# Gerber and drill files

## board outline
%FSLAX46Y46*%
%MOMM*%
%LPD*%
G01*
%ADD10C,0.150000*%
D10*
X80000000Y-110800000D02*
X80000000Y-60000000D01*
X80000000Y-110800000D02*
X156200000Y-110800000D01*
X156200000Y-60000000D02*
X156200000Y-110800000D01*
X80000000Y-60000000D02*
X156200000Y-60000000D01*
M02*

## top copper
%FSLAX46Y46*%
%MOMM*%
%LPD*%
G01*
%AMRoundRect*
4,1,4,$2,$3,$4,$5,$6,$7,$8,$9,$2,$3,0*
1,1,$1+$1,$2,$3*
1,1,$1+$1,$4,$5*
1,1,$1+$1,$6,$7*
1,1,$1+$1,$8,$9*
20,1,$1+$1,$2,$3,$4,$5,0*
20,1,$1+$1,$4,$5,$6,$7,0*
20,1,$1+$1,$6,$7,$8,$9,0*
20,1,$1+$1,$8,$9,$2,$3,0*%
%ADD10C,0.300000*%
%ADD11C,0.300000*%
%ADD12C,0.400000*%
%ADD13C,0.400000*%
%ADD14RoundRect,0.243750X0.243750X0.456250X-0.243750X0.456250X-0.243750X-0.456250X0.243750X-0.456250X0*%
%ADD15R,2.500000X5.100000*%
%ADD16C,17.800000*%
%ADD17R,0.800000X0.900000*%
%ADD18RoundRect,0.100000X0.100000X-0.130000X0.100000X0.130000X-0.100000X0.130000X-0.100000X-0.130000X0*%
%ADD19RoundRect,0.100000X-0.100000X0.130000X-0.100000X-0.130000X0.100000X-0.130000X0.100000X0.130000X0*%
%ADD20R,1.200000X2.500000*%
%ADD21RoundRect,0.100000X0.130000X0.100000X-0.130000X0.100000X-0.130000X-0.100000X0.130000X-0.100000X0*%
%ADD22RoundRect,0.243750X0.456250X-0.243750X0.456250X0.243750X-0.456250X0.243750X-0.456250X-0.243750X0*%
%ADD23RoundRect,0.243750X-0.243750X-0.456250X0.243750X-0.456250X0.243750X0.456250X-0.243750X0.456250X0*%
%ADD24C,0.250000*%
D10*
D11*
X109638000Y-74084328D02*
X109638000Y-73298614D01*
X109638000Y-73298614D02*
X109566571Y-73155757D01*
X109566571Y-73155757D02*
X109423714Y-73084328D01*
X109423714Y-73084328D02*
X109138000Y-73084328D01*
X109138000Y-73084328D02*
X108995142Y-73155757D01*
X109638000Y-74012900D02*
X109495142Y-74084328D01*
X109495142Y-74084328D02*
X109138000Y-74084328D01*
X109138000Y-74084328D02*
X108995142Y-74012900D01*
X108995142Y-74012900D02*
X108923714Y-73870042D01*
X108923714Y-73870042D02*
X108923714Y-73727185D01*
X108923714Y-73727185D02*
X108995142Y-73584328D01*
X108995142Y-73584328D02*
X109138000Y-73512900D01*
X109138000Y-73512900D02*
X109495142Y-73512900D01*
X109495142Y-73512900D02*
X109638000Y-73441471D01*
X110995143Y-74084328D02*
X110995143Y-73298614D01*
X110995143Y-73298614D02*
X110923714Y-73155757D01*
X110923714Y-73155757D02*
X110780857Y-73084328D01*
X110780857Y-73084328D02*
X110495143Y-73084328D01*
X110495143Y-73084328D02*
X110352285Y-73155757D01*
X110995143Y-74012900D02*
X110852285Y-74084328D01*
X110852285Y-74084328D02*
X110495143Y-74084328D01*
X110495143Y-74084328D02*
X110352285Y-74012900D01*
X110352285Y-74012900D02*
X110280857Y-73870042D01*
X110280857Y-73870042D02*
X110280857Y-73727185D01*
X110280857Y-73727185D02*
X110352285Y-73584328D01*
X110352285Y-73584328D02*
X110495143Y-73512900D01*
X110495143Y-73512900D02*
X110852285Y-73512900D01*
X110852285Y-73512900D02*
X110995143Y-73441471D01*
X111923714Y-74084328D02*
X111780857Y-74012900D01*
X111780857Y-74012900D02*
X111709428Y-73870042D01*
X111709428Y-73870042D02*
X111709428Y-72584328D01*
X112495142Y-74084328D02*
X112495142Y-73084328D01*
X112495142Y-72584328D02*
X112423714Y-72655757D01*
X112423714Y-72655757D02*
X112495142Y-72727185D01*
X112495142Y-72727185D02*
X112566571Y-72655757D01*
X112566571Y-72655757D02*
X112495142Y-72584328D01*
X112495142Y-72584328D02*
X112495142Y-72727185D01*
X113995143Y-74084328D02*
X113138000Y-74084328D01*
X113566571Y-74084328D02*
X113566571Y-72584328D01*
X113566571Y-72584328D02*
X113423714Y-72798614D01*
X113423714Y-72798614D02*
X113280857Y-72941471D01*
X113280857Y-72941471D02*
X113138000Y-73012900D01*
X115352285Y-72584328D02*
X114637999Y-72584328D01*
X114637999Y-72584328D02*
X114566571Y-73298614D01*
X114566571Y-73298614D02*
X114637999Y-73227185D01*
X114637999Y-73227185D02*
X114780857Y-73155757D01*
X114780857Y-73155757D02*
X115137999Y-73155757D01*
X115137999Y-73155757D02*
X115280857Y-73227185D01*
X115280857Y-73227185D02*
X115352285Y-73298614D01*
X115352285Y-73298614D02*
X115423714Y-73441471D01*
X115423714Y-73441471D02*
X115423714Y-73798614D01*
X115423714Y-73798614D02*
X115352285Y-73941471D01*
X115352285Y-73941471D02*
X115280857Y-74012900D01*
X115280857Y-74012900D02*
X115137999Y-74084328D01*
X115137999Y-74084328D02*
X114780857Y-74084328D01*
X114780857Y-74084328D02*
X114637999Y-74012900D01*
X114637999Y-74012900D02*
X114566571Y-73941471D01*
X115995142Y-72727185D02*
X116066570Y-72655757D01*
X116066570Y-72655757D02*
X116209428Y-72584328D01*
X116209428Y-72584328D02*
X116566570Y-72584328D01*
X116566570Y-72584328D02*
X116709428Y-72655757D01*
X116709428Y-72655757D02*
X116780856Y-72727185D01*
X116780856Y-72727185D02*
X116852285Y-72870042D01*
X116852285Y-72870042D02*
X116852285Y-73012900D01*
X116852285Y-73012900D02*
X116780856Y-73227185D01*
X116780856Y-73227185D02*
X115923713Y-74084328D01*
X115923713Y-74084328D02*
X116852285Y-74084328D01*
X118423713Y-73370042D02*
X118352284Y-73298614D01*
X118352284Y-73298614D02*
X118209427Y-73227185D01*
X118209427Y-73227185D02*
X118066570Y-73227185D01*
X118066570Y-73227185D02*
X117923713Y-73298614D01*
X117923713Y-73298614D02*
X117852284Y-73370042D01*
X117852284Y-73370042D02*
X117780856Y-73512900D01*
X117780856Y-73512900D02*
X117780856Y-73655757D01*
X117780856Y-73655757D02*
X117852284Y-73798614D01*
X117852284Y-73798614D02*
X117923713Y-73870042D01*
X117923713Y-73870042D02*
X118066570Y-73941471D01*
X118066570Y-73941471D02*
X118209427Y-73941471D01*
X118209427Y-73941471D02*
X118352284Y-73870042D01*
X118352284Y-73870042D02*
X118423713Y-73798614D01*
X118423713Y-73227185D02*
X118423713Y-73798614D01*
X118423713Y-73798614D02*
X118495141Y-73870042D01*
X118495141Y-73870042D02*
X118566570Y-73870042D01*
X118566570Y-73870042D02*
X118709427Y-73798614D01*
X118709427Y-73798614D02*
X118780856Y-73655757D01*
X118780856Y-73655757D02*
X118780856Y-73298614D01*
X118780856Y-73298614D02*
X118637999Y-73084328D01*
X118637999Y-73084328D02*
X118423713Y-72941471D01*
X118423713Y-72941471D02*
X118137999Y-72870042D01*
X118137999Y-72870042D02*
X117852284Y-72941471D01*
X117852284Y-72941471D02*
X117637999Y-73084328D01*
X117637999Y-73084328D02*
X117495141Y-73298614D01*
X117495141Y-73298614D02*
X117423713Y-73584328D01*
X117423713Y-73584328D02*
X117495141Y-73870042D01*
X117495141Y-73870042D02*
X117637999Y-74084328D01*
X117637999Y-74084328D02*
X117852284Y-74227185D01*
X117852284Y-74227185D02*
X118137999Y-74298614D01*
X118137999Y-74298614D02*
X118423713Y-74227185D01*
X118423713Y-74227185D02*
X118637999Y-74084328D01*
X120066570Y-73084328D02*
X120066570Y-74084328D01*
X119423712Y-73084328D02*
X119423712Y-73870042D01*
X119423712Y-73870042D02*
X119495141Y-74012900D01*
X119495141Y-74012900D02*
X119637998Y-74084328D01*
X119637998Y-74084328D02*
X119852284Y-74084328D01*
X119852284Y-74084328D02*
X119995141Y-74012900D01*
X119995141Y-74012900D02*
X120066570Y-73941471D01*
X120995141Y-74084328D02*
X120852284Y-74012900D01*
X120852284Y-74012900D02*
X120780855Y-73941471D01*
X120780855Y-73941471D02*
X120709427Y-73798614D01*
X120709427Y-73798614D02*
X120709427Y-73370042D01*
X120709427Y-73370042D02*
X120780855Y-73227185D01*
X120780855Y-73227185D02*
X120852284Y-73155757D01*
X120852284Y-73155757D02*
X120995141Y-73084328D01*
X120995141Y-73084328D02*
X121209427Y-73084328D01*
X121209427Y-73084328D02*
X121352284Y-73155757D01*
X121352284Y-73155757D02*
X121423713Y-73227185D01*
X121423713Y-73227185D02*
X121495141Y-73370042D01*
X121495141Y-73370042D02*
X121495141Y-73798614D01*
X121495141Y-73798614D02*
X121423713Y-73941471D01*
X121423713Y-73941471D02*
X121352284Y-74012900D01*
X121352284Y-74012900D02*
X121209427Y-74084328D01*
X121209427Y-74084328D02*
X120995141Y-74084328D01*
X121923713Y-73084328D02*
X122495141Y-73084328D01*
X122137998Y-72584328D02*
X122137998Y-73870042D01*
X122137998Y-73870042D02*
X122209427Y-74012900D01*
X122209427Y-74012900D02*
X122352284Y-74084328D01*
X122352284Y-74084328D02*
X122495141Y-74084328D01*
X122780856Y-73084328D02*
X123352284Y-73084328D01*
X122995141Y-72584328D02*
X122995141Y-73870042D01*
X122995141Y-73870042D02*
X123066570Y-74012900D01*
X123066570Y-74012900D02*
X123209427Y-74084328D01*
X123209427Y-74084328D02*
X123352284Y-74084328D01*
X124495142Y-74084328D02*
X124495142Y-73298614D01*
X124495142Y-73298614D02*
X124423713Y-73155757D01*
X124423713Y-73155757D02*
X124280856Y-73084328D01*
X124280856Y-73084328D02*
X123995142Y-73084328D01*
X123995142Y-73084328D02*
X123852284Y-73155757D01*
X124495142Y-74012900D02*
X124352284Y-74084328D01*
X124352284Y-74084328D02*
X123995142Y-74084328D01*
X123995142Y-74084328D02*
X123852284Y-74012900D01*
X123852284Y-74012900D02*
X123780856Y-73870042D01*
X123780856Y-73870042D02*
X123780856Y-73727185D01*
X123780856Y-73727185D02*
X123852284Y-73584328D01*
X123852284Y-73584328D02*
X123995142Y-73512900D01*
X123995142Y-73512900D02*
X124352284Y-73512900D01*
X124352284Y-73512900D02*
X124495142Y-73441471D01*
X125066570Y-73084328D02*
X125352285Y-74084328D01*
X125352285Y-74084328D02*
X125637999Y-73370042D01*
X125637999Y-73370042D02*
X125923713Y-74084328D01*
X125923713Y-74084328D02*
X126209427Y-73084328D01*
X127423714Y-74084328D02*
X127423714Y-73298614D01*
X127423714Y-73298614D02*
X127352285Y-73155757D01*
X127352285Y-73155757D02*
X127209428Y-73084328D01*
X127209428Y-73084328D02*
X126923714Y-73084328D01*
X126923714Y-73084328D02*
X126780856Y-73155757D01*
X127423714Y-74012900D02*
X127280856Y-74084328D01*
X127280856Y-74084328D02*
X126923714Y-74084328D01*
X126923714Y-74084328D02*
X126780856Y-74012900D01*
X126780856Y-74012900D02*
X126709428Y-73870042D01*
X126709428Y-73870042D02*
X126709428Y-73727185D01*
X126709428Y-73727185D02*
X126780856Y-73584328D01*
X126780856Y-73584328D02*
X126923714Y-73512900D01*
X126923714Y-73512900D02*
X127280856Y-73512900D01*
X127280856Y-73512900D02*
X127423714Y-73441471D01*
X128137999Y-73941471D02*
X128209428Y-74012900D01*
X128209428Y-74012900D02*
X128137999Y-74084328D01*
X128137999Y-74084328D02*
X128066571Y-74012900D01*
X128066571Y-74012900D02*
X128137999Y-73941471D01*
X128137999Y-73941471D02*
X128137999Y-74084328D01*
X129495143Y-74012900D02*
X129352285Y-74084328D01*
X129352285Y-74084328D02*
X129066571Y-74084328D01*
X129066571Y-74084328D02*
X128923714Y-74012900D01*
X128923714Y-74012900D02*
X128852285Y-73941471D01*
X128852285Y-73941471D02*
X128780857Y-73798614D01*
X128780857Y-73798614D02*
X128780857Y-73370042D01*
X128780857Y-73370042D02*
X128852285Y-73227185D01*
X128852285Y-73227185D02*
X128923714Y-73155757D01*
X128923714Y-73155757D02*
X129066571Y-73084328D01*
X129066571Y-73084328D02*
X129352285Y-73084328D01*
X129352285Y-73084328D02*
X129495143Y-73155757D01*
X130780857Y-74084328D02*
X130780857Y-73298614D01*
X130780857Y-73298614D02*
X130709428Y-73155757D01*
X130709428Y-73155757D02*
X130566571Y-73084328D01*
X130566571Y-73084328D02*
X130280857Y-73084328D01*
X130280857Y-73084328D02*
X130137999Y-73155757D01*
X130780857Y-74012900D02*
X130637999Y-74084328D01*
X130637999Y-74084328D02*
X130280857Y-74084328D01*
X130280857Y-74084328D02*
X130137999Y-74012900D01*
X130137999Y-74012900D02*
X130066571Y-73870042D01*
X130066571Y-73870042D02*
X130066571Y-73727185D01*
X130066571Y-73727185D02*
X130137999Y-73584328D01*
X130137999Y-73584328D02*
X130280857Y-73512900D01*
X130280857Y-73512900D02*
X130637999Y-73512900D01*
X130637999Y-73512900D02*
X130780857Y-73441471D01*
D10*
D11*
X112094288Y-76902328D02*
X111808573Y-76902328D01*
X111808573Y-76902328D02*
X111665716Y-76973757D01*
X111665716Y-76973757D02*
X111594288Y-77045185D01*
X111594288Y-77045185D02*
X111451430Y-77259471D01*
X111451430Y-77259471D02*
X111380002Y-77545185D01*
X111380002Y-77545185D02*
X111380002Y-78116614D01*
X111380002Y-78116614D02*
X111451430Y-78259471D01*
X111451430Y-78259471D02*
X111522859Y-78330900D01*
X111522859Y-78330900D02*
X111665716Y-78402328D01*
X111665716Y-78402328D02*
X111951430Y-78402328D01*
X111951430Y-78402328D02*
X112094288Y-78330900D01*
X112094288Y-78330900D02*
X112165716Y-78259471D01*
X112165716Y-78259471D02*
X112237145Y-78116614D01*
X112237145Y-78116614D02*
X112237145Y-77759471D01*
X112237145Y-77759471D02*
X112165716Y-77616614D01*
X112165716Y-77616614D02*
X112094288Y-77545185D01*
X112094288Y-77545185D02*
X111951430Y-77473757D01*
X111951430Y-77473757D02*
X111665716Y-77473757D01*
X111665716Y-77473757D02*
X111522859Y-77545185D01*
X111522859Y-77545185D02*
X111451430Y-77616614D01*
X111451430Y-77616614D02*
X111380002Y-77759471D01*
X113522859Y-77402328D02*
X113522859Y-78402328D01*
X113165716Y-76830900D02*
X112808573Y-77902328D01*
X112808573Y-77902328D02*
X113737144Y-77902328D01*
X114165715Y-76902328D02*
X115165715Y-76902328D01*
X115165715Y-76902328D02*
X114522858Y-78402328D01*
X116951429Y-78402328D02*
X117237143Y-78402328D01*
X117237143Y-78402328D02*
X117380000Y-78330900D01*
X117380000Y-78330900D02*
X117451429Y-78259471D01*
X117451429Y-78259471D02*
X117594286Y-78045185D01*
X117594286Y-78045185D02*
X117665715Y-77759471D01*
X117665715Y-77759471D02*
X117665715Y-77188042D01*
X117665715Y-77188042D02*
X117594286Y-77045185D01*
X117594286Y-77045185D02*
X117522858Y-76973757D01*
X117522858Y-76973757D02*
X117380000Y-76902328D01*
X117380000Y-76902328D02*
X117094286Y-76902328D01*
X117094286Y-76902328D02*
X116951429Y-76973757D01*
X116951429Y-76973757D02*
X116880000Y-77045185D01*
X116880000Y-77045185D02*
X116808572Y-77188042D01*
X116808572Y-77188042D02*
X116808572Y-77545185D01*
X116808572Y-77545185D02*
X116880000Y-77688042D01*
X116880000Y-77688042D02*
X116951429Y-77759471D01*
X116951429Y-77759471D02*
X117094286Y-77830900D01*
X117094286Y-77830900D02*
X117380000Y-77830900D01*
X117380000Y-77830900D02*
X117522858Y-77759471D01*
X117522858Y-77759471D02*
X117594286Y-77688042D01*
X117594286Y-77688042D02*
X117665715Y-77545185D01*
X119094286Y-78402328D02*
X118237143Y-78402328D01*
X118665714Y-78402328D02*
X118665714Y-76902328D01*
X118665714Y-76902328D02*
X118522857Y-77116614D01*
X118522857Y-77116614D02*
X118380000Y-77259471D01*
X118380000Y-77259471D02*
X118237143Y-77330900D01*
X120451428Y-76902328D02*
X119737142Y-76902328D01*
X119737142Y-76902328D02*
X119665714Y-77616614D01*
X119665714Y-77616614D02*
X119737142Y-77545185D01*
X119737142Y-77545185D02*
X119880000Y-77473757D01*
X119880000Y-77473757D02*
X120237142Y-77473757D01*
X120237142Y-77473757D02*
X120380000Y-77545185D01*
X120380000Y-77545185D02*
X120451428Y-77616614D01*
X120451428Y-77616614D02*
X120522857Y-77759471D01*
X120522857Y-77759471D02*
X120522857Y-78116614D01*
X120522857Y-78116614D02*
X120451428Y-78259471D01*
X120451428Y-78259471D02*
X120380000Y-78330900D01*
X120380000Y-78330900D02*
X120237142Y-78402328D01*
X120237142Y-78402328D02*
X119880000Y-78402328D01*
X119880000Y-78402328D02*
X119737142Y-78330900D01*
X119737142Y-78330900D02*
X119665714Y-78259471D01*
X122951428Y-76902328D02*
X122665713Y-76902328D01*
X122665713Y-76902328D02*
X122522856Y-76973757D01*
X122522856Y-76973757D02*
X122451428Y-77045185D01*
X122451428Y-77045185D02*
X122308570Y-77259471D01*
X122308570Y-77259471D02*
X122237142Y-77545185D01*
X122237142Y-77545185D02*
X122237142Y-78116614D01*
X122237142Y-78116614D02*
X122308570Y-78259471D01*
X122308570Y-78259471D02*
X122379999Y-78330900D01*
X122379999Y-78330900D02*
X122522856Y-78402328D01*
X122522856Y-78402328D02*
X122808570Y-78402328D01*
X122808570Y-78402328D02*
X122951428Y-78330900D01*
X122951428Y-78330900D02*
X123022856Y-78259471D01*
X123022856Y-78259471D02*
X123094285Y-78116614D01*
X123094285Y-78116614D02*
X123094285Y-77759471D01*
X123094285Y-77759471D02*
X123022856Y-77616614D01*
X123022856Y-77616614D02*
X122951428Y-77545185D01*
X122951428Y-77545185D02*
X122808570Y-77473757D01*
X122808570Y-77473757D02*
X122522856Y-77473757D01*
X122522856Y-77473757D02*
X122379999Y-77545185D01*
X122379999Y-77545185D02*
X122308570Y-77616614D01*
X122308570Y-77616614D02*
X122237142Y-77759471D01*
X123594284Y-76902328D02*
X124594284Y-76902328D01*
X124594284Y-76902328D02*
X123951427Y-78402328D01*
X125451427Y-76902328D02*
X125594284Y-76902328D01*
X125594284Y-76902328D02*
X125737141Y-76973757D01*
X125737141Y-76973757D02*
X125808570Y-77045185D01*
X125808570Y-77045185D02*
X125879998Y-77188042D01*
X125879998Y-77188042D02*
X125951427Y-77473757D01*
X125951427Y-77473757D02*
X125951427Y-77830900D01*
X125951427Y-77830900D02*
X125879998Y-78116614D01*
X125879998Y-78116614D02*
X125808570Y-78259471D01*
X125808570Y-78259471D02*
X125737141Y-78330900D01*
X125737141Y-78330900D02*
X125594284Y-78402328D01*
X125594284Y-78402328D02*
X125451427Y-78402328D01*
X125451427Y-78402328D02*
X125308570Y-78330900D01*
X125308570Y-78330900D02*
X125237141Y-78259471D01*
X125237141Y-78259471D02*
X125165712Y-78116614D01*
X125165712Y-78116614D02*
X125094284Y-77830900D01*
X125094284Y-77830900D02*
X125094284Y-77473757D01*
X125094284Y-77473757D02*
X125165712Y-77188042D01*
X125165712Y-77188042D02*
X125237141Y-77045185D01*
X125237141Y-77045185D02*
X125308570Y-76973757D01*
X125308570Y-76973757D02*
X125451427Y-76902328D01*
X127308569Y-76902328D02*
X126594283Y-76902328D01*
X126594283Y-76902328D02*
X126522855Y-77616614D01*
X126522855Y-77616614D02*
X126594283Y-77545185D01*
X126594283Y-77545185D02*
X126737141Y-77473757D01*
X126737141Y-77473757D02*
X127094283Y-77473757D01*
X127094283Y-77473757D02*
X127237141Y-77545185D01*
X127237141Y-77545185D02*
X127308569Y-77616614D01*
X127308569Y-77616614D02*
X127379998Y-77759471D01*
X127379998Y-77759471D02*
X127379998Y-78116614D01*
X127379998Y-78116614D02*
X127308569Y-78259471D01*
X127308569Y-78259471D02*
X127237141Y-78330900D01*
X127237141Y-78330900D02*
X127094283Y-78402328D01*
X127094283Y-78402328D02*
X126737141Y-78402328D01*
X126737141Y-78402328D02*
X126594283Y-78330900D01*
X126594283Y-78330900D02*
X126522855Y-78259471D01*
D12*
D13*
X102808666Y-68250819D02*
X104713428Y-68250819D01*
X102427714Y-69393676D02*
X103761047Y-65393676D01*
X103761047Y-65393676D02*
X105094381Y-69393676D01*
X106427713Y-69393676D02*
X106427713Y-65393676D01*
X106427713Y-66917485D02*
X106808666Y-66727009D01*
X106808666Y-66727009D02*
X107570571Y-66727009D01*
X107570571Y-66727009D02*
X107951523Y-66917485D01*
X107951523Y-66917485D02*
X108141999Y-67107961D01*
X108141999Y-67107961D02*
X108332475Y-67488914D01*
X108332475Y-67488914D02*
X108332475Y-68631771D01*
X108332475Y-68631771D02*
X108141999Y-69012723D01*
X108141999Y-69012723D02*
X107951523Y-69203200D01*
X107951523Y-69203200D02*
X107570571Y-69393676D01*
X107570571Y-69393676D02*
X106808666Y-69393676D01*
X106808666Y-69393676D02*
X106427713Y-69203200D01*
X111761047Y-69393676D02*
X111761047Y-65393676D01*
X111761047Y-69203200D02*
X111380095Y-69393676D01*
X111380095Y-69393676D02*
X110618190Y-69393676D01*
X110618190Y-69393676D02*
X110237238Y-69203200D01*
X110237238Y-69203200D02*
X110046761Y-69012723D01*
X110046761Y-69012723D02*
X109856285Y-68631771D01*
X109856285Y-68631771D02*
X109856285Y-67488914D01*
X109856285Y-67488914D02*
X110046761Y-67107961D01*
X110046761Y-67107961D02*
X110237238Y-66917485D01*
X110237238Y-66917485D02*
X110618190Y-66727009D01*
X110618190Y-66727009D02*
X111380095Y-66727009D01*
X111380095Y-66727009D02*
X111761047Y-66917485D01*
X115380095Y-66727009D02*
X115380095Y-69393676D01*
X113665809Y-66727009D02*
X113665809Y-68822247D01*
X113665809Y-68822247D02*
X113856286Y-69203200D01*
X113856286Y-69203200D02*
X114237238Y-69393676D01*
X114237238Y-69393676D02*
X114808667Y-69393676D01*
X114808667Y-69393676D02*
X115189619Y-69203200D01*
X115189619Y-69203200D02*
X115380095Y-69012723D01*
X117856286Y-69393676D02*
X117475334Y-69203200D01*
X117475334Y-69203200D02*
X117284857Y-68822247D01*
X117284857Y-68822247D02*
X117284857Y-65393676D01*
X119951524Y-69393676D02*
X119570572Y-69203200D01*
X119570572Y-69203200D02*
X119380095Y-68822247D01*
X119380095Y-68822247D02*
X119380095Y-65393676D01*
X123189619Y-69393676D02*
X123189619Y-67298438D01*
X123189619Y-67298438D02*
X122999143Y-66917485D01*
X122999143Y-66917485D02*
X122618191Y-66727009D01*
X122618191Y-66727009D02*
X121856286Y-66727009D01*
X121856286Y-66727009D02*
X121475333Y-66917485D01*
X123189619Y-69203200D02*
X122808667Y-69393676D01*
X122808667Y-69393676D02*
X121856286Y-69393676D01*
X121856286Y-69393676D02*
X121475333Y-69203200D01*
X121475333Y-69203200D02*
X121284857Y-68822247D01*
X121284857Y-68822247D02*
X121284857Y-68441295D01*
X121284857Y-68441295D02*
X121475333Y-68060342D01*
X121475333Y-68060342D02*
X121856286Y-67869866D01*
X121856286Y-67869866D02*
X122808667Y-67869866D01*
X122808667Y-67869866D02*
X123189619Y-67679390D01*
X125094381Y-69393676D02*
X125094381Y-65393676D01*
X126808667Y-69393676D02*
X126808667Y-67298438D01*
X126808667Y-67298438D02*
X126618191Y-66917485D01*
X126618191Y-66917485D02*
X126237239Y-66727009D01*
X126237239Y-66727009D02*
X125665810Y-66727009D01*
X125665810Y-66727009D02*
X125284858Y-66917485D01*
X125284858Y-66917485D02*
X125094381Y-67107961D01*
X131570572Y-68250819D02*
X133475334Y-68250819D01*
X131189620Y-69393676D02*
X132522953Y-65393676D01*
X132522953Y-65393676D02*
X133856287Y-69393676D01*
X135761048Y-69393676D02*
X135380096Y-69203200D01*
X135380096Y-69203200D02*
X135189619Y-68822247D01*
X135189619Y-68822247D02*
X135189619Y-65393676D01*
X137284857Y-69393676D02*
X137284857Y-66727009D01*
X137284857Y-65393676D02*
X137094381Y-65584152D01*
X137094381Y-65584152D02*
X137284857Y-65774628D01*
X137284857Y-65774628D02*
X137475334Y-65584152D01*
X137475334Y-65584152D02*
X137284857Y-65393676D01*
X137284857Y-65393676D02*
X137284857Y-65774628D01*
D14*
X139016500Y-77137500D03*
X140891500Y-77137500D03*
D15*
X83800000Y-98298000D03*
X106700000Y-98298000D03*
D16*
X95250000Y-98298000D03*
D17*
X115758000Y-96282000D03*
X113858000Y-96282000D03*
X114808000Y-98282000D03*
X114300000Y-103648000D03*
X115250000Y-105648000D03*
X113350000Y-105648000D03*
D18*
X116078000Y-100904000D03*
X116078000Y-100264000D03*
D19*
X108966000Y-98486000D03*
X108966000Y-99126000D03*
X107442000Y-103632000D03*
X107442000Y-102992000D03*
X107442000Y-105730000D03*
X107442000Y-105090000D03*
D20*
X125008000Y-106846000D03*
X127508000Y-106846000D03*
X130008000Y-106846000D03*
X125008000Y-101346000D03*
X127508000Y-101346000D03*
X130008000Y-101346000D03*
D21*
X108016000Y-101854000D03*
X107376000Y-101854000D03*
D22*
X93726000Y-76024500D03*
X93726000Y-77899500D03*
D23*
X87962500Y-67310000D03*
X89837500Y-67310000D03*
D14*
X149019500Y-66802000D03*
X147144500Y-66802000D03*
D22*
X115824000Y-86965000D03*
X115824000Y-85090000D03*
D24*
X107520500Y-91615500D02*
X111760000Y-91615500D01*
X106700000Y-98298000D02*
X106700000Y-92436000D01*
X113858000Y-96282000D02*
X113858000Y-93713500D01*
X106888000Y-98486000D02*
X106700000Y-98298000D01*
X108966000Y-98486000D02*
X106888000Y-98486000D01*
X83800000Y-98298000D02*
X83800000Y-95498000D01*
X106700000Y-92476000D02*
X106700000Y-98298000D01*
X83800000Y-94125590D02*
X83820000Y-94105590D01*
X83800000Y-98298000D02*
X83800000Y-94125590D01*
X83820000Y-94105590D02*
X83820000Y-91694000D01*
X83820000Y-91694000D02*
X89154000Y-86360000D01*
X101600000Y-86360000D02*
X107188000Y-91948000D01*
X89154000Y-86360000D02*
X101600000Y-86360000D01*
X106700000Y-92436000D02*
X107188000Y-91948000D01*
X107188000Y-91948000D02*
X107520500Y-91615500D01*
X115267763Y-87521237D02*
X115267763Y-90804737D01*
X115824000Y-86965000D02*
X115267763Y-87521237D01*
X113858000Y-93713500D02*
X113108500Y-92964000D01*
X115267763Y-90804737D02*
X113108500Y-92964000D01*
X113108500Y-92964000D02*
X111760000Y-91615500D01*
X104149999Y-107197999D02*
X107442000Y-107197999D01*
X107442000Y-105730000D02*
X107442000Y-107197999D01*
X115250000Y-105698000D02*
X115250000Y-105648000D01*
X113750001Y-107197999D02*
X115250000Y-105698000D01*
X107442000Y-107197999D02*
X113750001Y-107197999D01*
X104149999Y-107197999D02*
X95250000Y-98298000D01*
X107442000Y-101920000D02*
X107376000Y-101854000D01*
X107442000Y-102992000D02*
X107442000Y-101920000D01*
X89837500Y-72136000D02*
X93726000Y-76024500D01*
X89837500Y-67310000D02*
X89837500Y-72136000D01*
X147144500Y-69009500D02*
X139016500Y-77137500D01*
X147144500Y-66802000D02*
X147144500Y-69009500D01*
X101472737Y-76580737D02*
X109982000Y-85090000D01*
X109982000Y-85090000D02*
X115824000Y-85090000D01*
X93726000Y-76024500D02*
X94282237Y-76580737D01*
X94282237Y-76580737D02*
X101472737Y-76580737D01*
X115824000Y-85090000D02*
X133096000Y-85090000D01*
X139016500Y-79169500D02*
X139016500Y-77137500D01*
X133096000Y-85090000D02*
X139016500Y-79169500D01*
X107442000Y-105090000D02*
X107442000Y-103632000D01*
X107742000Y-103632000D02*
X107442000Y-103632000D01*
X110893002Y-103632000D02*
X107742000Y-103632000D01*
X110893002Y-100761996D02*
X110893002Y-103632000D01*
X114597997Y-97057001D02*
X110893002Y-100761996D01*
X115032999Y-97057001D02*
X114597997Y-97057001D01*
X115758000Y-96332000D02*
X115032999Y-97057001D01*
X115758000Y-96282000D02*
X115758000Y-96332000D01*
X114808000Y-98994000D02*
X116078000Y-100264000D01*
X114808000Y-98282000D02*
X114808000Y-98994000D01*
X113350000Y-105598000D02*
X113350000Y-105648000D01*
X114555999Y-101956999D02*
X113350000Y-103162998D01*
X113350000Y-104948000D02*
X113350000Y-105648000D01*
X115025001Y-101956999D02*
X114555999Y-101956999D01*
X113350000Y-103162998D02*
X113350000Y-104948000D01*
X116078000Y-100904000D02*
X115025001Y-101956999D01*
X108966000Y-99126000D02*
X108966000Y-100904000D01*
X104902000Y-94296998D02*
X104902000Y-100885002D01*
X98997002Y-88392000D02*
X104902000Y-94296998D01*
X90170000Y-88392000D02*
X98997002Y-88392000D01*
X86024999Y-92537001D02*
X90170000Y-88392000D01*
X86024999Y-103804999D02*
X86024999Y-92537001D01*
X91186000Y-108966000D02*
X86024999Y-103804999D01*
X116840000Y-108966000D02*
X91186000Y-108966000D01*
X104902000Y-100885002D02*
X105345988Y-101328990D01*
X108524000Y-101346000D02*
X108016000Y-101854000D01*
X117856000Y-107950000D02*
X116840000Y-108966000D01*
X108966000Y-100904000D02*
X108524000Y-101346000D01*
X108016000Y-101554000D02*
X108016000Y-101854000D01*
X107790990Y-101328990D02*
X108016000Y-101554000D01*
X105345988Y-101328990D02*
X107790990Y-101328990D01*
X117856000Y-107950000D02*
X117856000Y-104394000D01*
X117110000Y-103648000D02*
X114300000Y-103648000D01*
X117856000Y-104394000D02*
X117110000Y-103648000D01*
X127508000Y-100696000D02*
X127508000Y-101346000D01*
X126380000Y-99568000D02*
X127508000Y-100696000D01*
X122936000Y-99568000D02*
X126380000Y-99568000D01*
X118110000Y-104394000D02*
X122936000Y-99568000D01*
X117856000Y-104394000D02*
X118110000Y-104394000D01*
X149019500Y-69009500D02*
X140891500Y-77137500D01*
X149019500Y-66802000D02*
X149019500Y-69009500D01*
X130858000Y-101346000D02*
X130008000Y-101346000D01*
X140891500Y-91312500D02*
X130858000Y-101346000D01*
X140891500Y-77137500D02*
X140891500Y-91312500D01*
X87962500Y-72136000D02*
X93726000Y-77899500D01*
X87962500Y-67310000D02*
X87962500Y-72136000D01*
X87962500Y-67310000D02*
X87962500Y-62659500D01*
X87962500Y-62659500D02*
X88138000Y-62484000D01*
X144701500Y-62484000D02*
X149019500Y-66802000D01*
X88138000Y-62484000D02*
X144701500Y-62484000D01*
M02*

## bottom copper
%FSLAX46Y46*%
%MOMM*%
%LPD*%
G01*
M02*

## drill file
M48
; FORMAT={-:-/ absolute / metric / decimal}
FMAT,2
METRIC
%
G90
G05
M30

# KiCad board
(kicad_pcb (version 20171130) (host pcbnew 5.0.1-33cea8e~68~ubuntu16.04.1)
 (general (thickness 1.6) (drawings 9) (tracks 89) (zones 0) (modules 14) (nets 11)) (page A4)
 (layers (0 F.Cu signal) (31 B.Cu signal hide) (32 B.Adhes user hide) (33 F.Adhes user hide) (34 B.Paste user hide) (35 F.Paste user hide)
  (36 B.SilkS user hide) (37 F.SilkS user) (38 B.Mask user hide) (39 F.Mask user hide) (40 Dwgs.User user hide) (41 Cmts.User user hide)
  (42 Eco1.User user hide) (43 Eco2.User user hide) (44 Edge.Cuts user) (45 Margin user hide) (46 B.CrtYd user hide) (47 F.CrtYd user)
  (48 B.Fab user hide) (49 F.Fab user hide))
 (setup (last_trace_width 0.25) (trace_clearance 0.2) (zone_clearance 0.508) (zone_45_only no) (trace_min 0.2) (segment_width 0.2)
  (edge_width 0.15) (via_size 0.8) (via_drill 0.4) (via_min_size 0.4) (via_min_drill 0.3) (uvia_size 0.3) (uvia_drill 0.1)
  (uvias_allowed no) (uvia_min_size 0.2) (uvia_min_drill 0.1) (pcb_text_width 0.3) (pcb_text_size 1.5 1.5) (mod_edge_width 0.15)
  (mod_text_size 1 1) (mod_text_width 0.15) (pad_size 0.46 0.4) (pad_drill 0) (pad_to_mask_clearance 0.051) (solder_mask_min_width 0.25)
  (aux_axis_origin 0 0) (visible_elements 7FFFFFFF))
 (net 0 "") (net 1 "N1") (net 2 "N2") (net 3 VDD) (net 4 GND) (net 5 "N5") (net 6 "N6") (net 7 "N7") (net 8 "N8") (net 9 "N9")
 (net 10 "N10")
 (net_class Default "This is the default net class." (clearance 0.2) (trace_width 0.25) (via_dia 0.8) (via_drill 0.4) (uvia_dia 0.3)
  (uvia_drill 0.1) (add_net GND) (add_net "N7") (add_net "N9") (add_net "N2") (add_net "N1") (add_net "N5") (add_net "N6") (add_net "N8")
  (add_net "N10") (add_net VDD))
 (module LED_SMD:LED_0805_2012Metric (layer F.Cu) (at 139.954 77.1375 180)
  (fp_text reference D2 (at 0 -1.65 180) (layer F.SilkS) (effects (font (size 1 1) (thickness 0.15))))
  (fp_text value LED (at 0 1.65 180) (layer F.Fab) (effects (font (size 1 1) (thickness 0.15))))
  (pad 2 smd roundrect (at 0.9375 0 180) (size 0.975 1.4) (layers F.Cu F.Paste F.Mask) (roundrect_rratio 0.25) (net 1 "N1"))
  (pad 1 smd roundrect (at -0.9375 0 180) (size 0.975 1.4) (layers F.Cu F.Paste F.Mask) (roundrect_rratio 0.25) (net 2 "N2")))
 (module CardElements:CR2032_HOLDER (layer F.Cu) (at 95.25 98.298)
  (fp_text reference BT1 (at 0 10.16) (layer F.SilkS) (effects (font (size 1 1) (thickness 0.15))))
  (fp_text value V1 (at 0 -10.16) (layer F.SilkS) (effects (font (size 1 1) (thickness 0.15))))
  (pad 1 smd rect (at -11.45 0) (size 2.5 5.1) (layers F.Cu F.Paste F.Mask) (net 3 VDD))
  (pad 1 smd rect (at 11.45 0) (size 2.5 5.1) (layers F.Cu F.Paste F.Mask) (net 3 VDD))
  (pad 2 smd circle (at 0 0) (size 17.8 17.8) (layers F.Cu F.Paste F.Mask) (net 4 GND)))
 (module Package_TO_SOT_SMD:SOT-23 (layer F.Cu) (at 114.808 97.282 270)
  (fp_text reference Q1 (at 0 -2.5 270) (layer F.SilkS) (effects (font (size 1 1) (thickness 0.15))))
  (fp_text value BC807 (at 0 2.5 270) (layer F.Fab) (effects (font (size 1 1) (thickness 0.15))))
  (pad 1 smd rect (at -1 -0.95 270) (size 0.9 0.8) (layers F.Cu F.Paste F.Mask) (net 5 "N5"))
  (pad 2 smd rect (at -1 0.95 270) (size 0.9 0.8) (layers F.Cu F.Paste F.Mask) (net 3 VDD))
  (pad 3 smd rect (at 1 0 270) (size 0.9 0.8) (layers F.Cu F.Paste F.Mask) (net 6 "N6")))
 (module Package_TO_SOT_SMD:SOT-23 (layer F.Cu) (at 114.3 104.648 90)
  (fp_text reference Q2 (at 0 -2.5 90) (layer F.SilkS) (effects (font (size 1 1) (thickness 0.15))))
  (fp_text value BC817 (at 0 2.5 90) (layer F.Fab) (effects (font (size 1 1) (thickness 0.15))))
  (pad 3 smd rect (at 1 0 90) (size 0.9 0.8) (layers F.Cu F.Paste F.Mask) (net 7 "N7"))
  (pad 2 smd rect (at -1 0.95 90) (size 0.9 0.8) (layers F.Cu F.Paste F.Mask) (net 4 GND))
  (pad 1 smd rect (at -1 -0.95 90) (size 0.9 0.8) (layers F.Cu F.Paste F.Mask) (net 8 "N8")))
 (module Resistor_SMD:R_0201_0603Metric (layer F.Cu) (at 116.078 100.584 90)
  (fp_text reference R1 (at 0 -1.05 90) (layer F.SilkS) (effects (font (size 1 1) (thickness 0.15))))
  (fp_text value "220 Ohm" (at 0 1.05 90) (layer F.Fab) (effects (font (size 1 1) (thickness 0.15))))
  (pad "" smd roundrect (at -0.345 0 90) (size 0.318 0.36) (layers F.Paste) (roundrect_rratio 0.25))
  (pad "" smd roundrect (at 0.345 0 90) (size 0.318 0.36) (layers F.Paste) (roundrect_rratio 0.25))
  (pad 1 smd roundrect (at -0.32 0 90) (size 0.46 0.4) (layers F.Cu F.Mask) (roundrect_rratio 0.25) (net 8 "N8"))
  (pad 2 smd roundrect (at 0.32 0 90) (size 0.46 0.4) (layers F.Cu F.Mask) (roundrect_rratio 0.25) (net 6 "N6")))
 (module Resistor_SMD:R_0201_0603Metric (layer F.Cu) (at 108.966 98.806 270)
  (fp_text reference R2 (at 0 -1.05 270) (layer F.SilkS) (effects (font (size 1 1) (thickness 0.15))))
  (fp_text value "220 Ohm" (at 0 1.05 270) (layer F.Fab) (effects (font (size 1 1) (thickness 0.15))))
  (pad "" smd roundrect (at -0.345 0 270) (size 0.318 0.36) (layers F.Paste) (roundrect_rratio 0.25))
  (pad "" smd roundrect (at 0.345 0 270) (size 0.318 0.36) (layers F.Paste) (roundrect_rratio 0.25))
  (pad 1 smd roundrect (at -0.32 0 270) (size 0.46 0.4) (layers F.Cu F.Mask) (roundrect_rratio 0.25) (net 3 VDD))
  (pad 2 smd roundrect (at 0.32 0 270) (size 0.46 0.4) (layers F.Cu F.Mask) (roundrect_rratio 0.25) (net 7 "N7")))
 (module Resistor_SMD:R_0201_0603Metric (layer F.Cu) (at 107.442 103.312 270)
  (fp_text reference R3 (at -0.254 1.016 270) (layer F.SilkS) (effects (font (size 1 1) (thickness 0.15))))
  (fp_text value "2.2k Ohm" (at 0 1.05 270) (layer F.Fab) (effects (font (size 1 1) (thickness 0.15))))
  (pad 2 smd roundrect (at 0.32 0 270) (size 0.46 0.4) (layers F.Cu F.Mask) (roundrect_rratio 0.25) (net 5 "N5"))
  (pad 1 smd roundrect (at -0.32 0 270) (size 0.46 0.4) (layers F.Cu F.Mask) (roundrect_rratio 0.25) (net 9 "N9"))
  (pad "" smd roundrect (at 0.345 0 270) (size 0.318 0.36) (layers F.Paste) (roundrect_rratio 0.25))
  (pad "" smd roundrect (at -0.345 0 270) (size 0.318 0.36) (layers F.Paste) (roundrect_rratio 0.25)))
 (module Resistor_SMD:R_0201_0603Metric (layer F.Cu) (at 107.442 105.41 270)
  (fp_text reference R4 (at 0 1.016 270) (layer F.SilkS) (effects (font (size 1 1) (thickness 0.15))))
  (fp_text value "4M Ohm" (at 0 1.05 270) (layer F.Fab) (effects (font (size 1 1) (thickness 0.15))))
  (pad 2 smd roundrect (at 0.32 0 270) (size 0.46 0.4) (layers F.Cu F.Mask) (roundrect_rratio 0.25) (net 4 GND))
  (pad 1 smd roundrect (at -0.32 0 270) (size 0.46 0.4) (layers F.Cu F.Mask) (roundrect_rratio 0.25) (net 5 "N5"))
  (pad "" smd roundrect (at 0.345 0 270) (size 0.318 0.36) (layers F.Paste) (roundrect_rratio 0.25))
  (pad "" smd roundrect (at -0.345 0 270) (size 0.318 0.36) (layers F.Paste) (roundrect_rratio 0.25)))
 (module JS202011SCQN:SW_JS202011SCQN (layer F.Cu) (at 127.508 104.096 180)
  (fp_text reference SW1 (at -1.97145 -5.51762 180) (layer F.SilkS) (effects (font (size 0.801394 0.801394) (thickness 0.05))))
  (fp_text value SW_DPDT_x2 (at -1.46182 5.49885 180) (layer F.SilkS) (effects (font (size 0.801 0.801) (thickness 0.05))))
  (pad 6 smd rect (at 2.5 -2.75 180) (size 1.2 2.5) (layers F.Cu F.Paste F.Mask))
  (pad 5 smd rect (at 0 -2.75 180) (size 1.2 2.5) (layers F.Cu F.Paste F.Mask))
  (pad 4 smd rect (at -2.5 -2.75 180) (size 1.2 2.5) (layers F.Cu F.Paste F.Mask))
  (pad 3 smd rect (at 2.5 2.75 180) (size 1.2 2.5) (layers F.Cu F.Paste F.Mask) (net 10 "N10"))
  (pad 2 smd rect (at 0 2.75 180) (size 1.2 2.5) (layers F.Cu F.Paste F.Mask) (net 7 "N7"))
  (pad 1 smd rect (at -2.5 2.75 180) (size 1.2 2.5) (layers F.Cu F.Paste F.Mask) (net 2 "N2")))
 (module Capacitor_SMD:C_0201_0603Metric (layer F.Cu) (at 107.696 101.854 180)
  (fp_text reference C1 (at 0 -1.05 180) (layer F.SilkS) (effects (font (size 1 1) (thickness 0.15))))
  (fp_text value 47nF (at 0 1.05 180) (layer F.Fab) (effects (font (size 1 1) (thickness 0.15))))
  (pad "" smd roundrect (at -0.345 0 180) (size 0.318 0.36) (layers F.Paste) (roundrect_rratio 0.25))
  (pad "" smd roundrect (at 0.345 0 180) (size 0.318 0.36) (layers F.Paste) (roundrect_rratio 0.25))
  (pad 1 smd roundrect (at -0.32 0 180) (size 0.46 0.4) (layers F.Cu F.Mask) (roundrect_rratio 0.25) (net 7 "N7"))
  (pad 2 smd roundrect (at 0.32 0 180) (size 0.46 0.4) (layers F.Cu F.Mask) (roundrect_rratio 0.25) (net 9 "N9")))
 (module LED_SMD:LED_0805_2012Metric (layer F.Cu) (at 93.726 76.962 90)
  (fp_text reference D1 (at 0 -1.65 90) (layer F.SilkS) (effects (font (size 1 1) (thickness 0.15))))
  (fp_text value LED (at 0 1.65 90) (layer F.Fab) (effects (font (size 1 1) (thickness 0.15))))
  (pad 2 smd roundrect (at 0.9375 0 90) (size 0.975 1.4) (layers F.Cu F.Paste F.Mask) (roundrect_rratio 0.25) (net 1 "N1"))
  (pad 1 smd roundrect (at -0.9375 0 90) (size 0.975 1.4) (layers F.Cu F.Paste F.Mask) (roundrect_rratio 0.25) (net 2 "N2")))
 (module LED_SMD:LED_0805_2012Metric (layer F.Cu) (at 88.9 67.31)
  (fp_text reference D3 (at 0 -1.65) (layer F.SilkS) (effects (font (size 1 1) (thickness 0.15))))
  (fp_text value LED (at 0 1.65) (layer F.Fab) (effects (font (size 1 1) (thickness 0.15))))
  (pad 1 smd roundrect (at -0.9375 0) (size 0.975 1.4) (layers F.Cu F.Paste F.Mask) (roundrect_rratio 0.25) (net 2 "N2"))
  (pad 2 smd roundrect (at 0.9375 0) (size 0.975 1.4) (layers F.Cu F.Paste F.Mask) (roundrect_rratio 0.25) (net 1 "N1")))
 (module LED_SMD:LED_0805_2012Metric (layer F.Cu) (at 148.082 66.802 180)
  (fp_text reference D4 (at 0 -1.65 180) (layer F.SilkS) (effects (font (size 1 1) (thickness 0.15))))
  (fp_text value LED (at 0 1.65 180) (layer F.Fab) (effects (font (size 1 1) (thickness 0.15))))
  (pad 1 smd roundrect (at -0.9375 0 180) (size 0.975 1.4) (layers F.Cu F.Paste F.Mask) (roundrect_rratio 0.25) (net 2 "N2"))
  (pad 2 smd roundrect (at 0.9375 0 180) (size 0.975 1.4) (layers F.Cu F.Paste F.Mask) (roundrect_rratio 0.25) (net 1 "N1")))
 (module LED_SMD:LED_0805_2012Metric (layer F.Cu) (at 115.824 86.0275 90)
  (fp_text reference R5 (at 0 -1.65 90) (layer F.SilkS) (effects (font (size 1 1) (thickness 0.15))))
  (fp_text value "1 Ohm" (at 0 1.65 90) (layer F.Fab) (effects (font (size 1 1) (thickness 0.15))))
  (pad 1 smd roundrect (at -0.9375 0 90) (size 0.975 1.4) (layers F.Cu F.Paste F.Mask) (roundrect_rratio 0.25) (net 3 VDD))
  (pad 2 smd roundrect (at 0.9375 0 90) (size 0.975 1.4) (layers F.Cu F.Paste F.Mask) (roundrect_rratio 0.25) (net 1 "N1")))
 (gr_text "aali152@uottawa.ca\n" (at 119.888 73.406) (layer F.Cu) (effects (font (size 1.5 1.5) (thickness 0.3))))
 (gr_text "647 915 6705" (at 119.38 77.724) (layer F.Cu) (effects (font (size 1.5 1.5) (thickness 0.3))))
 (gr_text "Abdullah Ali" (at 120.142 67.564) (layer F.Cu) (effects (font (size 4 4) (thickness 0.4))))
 (gr_line (start 80 110.8) (end 80 60) (layer Edge.Cuts) (width 0.15))
 (gr_line (start 80 110.8) (end 156.2 110.8) (layer Edge.Cuts) (width 0.15))
 (gr_line (start 156.2 60) (end 156.2 110.8) (layer Edge.Cuts) (width 0.15))
 (gr_line (start 80 60) (end 156.2 60) (layer Edge.Cuts) (width 0.15))
 (segment (start 107.5205 91.6155) (end 111.76 91.6155) (width 0.25) (layer F.Cu) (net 3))
 (segment (start 106.7 98.298) (end 106.7 92.436) (width 0.25) (layer F.Cu) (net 3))
 (segment (start 113.858 96.282) (end 113.858 93.7135) (width 0.25) (layer F.Cu) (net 3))
 (segment (start 106.888 98.486) (end 106.7 98.298) (width 0.25) (layer F.Cu) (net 3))
 (segment (start 108.966 98.486) (end 106.888 98.486) (width 0.25) (layer F.Cu) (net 3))
 (segment (start 83.8 98.298) (end 83.8 95.498) (width 0.25) (layer F.Cu) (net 3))
 (segment (start 106.7 92.476) (end 106.7 98.298) (width 0.25) (layer F.Cu) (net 3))
 (segment (start 83.8 94.12559) (end 83.82 94.10559) (width 0.25) (layer F.Cu) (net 3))
 (segment (start 83.8 98.298) (end 83.8 94.12559) (width 0.25) (layer F.Cu) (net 3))
 (segment (start 83.82 94.10559) (end 83.82 91.694) (width 0.25) (layer F.Cu) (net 3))
 (segment (start 83.82 91.694) (end 89.154 86.36) (width 0.25) (layer F.Cu) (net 3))
 (segment (start 101.6 86.36) (end 107.188 91.948) (width 0.25) (layer F.Cu) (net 3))
 (segment (start 89.154 86.36) (end 101.6 86.36) (width 0.25) (layer F.Cu) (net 3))
 (segment (start 106.7 92.436) (end 107.188 91.948) (width 0.25) (layer F.Cu) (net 3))
 (segment (start 107.188 91.948) (end 107.5205 91.6155) (width 0.25) (layer F.Cu) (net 3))
 (segment (start 115.267763 87.521237) (end 115.267763 90.804737) (width 0.25) (layer F.Cu) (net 3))
 (segment (start 115.824 86.965) (end 115.267763 87.521237) (width 0.25) (layer F.Cu) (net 3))
 (segment (start 113.858 93.7135) (end 113.1085 92.964) (width 0.25) (layer F.Cu) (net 3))
 (segment (start 115.267763 90.804737) (end 113.1085 92.964) (width 0.25) (layer F.Cu) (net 3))
 (segment (start 113.1085 92.964) (end 111.76 91.6155) (width 0.25) (layer F.Cu) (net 3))
 (segment (start 104.149999 107.197999) (end 107.442 107.197999) (width 0.25) (layer F.Cu) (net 4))
 (segment (start 107.442 105.73) (end 107.442 107.197999) (width 0.25) (layer F.Cu) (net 4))
 (segment (start 115.25 105.698) (end 115.25 105.648) (width 0.25) (layer F.Cu) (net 4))
 (segment (start 113.750001 107.197999) (end 115.25 105.698) (width 0.25) (layer F.Cu) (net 4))
 (segment (start 107.442 107.197999) (end 113.750001 107.197999) (width 0.25) (layer F.Cu) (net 4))
 (segment (start 104.149999 107.197999) (end 95.25 98.298) (width 0.25) (layer F.Cu) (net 4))
 (segment (start 107.442 101.92) (end 107.376 101.854) (width 0.25) (layer F.Cu) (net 9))
 (segment (start 107.442 102.992) (end 107.442 101.92) (width 0.25) (layer F.Cu) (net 9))
 (segment (start 89.8375 72.136) (end 93.726 76.0245) (width 0.25) (layer F.Cu) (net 1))
 (segment (start 89.8375 67.31) (end 89.8375 72.136) (width 0.25) (layer F.Cu) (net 1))
 (segment (start 147.1445 69.0095) (end 139.0165 77.1375) (width 0.25) (layer F.Cu) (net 1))
 (segment (start 147.1445 66.802) (end 147.1445 69.0095) (width 0.25) (layer F.Cu) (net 1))
 (segment (start 101.472737 76.580737) (end 109.982 85.09) (width 0.25) (layer F.Cu) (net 1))
 (segment (start 109.982 85.09) (end 115.824 85.09) (width 0.25) (layer F.Cu) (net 1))
 (segment (start 93.726 76.0245) (end 94.282237 76.580737) (width 0.25) (layer F.Cu) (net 1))
 (segment (start 94.282237 76.580737) (end 101.472737 76.580737) (width 0.25) (layer F.Cu) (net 1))
 (segment (start 115.824 85.09) (end 133.096 85.09) (width 0.25) (layer F.Cu) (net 1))
 (segment (start 139.0165 79.1695) (end 139.0165 77.1375) (width 0.25) (layer F.Cu) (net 1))
 (segment (start 133.096 85.09) (end 139.0165 79.1695) (width 0.25) (layer F.Cu) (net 1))
 (segment (start 107.442 105.09) (end 107.442 103.632) (width 0.25) (layer F.Cu) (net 5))
 (segment (start 107.742 103.632) (end 107.442 103.632) (width 0.25) (layer F.Cu) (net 5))
 (segment (start 110.893002 103.632) (end 107.742 103.632) (width 0.25) (layer F.Cu) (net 5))
 (segment (start 110.893002 100.761996) (end 110.893002 103.632) (width 0.25) (layer F.Cu) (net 5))
 (segment (start 114.597997 97.057001) (end 110.893002 100.761996) (width 0.25) (layer F.Cu) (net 5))
 (segment (start 115.032999 97.057001) (end 114.597997 97.057001) (width 0.25) (layer F.Cu) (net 5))
 (segment (start 115.758 96.332) (end 115.032999 97.057001) (width 0.25) (layer F.Cu) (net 5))
 (segment (start 115.758 96.282) (end 115.758 96.332) (width 0.25) (layer F.Cu) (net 5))
 (segment (start 114.808 98.994) (end 116.078 100.264) (width 0.25) (layer F.Cu) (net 6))
 (segment (start 114.808 98.282) (end 114.808 98.994) (width 0.25) (layer F.Cu) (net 6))
 (segment (start 113.35 105.598) (end 113.35 105.648) (width 0.25) (layer F.Cu) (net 8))
 (segment (start 114.555999 101.956999) (end 113.35 103.162998) (width 0.25) (layer F.Cu) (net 8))
 (segment (start 113.35 104.948) (end 113.35 105.648) (width 0.25) (layer F.Cu) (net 8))
 (segment (start 115.025001 101.956999) (end 114.555999 101.956999) (width 0.25) (layer F.Cu) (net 8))
 (segment (start 113.35 103.162998) (end 113.35 104.948) (width 0.25) (layer F.Cu) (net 8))
 (segment (start 116.078 100.904) (end 115.025001 101.956999) (width 0.25) (layer F.Cu) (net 8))
 (segment (start 108.966 99.126) (end 108.966 100.904) (width 0.25) (layer F.Cu) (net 7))
 (segment (start 104.902 94.296998) (end 104.902 100.885002) (width 0.25) (layer F.Cu) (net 7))
 (segment (start 98.997002 88.392) (end 104.902 94.296998) (width 0.25) (layer F.Cu) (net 7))
 (segment (start 90.17 88.392) (end 98.997002 88.392) (width 0.25) (layer F.Cu) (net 7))
 (segment (start 86.024999 92.537001) (end 90.17 88.392) (width 0.25) (layer F.Cu) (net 7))
 (segment (start 86.024999 103.804999) (end 86.024999 92.537001) (width 0.25) (layer F.Cu) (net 7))
 (segment (start 91.186 108.966) (end 86.024999 103.804999) (width 0.25) (layer F.Cu) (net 7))
 (segment (start 116.84 108.966) (end 91.186 108.966) (width 0.25) (layer F.Cu) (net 7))
 (segment (start 104.902 100.885002) (end 105.345988 101.32899) (width 0.25) (layer F.Cu) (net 7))
 (segment (start 108.524 101.346) (end 108.016 101.854) (width 0.25) (layer F.Cu) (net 7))
 (segment (start 117.856 107.95) (end 116.84 108.966) (width 0.25) (layer F.Cu) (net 7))
 (segment (start 108.966 100.904) (end 108.524 101.346) (width 0.25) (layer F.Cu) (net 7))
 (segment (start 108.016 101.554) (end 108.016 101.854) (width 0.25) (layer F.Cu) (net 7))
 (segment (start 107.79099 101.32899) (end 108.016 101.554) (width 0.25) (layer F.Cu) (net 7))
 (segment (start 105.345988 101.32899) (end 107.79099 101.32899) (width 0.25) (layer F.Cu) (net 7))
 (segment (start 117.856 107.95) (end 117.856 104.394) (width 0.25) (layer F.Cu) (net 7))
 (segment (start 117.11 103.648) (end 114.3 103.648) (width 0.25) (layer F.Cu) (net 7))
 (segment (start 117.856 104.394) (end 117.11 103.648) (width 0.25) (layer F.Cu) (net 7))
 (segment (start 127.508 100.696) (end 127.508 101.346) (width 0.25) (layer F.Cu) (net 7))
 (segment (start 126.38 99.568) (end 127.508 100.696) (width 0.25) (layer F.Cu) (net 7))
 (segment (start 122.936 99.568) (end 126.38 99.568) (width 0.25) (layer F.Cu) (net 7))
 (segment (start 118.11 104.394) (end 122.936 99.568) (width 0.25) (layer F.Cu) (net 7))
 (segment (start 117.856 104.394) (end 118.11 104.394) (width 0.25) (layer F.Cu) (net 7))
 (segment (start 149.0195 69.0095) (end 140.8915 77.1375) (width 0.25) (layer F.Cu) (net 2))
 (segment (start 149.0195 66.802) (end 149.0195 69.0095) (width 0.25) (layer F.Cu) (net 2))
 (segment (start 130.858 101.346) (end 130.008 101.346) (width 0.25) (layer F.Cu) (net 2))
 (segment (start 140.8915 91.3125) (end 130.858 101.346) (width 0.25) (layer F.Cu) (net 2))
 (segment (start 140.8915 77.1375) (end 140.8915 91.3125) (width 0.25) (layer F.Cu) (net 2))
 (segment (start 87.9625 72.136) (end 93.726 77.8995) (width 0.25) (layer F.Cu) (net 2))
 (segment (start 87.9625 67.31) (end 87.9625 72.136) (width 0.25) (layer F.Cu) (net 2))
 (segment (start 87.9625 67.31) (end 87.9625 62.6595) (width 0.25) (layer F.Cu) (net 2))
 (segment (start 87.9625 62.6595) (end 88.138 62.484) (width 0.25) (layer F.Cu) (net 2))
 (segment (start 144.7015 62.484) (end 149.0195 66.802) (width 0.25) (layer F.Cu) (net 2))
 (segment (start 88.138 62.484) (end 144.7015 62.484) (width 0.25) (layer F.Cu) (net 2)))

